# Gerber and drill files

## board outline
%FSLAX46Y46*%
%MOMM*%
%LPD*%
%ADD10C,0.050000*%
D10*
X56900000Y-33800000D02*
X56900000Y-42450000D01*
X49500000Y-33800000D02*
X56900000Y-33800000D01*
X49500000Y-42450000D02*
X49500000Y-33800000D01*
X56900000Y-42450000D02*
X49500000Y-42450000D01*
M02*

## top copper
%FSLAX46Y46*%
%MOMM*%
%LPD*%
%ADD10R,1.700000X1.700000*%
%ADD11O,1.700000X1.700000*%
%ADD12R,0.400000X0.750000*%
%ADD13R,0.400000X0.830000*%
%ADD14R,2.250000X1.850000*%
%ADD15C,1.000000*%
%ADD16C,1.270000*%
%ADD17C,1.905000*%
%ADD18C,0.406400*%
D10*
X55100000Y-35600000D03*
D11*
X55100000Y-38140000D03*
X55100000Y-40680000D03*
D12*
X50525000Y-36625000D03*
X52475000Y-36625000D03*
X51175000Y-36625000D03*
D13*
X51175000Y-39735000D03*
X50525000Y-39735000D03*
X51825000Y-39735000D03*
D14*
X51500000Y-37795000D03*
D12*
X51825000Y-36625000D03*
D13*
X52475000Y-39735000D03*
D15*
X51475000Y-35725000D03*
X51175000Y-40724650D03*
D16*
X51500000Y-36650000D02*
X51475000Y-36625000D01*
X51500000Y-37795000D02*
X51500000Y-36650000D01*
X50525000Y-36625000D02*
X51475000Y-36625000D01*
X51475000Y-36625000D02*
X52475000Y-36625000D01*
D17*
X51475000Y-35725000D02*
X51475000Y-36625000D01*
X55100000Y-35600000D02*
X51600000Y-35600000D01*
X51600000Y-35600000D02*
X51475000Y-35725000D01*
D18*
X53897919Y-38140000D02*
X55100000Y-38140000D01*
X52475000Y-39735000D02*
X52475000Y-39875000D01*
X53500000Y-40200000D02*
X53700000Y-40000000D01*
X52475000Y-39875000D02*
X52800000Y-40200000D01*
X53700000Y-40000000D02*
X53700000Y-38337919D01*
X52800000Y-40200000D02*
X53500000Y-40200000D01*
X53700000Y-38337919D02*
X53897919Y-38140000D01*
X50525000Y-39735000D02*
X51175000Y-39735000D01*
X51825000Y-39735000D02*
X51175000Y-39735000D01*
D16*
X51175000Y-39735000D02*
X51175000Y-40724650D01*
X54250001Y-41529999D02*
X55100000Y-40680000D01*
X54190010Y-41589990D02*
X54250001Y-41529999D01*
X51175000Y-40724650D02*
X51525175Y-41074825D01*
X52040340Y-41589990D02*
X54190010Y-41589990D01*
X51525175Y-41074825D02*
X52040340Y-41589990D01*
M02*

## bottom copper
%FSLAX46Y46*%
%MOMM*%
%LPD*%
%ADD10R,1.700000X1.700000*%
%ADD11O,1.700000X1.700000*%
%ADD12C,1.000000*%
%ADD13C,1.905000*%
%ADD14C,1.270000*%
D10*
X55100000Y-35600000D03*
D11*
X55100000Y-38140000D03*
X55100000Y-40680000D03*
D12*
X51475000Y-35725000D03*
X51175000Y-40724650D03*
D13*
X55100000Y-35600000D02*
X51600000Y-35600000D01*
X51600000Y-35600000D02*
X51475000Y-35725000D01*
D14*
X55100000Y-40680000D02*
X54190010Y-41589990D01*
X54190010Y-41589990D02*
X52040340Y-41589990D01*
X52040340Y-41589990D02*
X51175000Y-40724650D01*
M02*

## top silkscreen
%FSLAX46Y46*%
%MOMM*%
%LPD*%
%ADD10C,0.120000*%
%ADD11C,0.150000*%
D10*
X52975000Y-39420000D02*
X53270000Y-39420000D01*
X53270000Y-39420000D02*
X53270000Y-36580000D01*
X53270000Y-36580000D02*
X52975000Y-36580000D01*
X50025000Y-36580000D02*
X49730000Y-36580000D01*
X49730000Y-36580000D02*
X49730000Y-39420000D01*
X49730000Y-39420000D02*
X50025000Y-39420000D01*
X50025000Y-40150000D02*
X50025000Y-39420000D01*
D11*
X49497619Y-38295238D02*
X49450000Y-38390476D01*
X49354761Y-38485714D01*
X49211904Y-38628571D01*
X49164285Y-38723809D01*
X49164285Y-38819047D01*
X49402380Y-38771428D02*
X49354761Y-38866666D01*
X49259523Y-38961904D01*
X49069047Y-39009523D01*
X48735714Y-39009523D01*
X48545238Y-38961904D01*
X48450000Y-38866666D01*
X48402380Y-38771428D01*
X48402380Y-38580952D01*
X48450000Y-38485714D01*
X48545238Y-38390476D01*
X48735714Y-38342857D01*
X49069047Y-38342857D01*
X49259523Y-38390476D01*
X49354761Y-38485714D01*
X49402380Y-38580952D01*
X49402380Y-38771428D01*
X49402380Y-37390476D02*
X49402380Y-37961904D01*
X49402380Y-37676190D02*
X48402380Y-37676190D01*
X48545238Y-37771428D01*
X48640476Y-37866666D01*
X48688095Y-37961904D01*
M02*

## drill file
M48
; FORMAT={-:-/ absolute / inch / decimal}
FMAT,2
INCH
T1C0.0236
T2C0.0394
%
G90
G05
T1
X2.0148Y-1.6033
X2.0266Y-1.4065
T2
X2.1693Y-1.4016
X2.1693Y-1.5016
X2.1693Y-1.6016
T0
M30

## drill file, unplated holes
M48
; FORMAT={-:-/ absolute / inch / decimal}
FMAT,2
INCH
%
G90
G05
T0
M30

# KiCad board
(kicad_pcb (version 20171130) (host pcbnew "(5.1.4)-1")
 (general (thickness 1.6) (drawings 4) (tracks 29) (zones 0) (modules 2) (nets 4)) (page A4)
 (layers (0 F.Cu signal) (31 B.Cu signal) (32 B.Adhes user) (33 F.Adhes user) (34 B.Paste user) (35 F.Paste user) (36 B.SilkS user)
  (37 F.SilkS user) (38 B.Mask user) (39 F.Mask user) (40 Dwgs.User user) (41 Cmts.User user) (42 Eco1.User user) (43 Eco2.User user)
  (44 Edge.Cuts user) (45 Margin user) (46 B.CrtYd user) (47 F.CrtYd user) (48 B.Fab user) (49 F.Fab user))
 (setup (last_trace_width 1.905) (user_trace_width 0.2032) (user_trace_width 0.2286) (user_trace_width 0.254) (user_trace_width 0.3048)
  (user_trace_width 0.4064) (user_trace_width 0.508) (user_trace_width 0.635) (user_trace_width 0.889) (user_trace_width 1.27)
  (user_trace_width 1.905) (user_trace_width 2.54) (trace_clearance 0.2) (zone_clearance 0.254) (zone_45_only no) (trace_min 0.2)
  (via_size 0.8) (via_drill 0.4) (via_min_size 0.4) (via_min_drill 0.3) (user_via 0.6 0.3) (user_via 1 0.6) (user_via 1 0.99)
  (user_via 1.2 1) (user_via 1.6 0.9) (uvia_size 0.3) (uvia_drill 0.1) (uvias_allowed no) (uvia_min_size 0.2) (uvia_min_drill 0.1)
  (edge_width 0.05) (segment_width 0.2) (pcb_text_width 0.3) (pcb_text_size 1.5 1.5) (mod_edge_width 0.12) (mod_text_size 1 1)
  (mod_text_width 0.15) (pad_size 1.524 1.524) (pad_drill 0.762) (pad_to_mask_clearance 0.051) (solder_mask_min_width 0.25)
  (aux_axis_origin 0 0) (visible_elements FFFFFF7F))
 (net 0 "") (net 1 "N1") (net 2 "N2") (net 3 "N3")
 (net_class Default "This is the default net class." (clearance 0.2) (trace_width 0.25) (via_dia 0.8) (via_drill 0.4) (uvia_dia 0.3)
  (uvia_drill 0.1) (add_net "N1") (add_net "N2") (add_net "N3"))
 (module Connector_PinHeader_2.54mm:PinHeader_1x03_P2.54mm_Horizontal (layer B.Cu) (at 55.1 35.6 180)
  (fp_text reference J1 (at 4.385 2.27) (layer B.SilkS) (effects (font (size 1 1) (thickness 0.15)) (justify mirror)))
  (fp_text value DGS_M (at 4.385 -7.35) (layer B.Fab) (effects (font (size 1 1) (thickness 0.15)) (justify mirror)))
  (pad 1 thru_hole rect (at 0 0 180) (size 1.7 1.7) (drill 1) (layers *.Cu *.Mask) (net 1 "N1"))
  (pad 2 thru_hole oval (at 0 -2.54 180) (size 1.7 1.7) (drill 1) (layers *.Cu *.Mask) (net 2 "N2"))
  (pad 3 thru_hole oval (at 0 -5.08 180) (size 1.7 1.7) (drill 1) (layers *.Cu *.Mask) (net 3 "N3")))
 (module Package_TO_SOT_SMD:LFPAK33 (layer F.Cu) (at 51.5 38.2 90) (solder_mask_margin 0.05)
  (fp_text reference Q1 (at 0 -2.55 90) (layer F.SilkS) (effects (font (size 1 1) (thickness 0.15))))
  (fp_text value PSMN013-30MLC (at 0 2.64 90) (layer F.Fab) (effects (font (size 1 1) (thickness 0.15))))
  (fp_line (start -1.22 1.475) (end -1.22 1.77) (layer F.SilkS) (width 0.12))
  (fp_line (start -1.22 1.77) (end 1.62 1.77) (layer F.SilkS) (width 0.12))
  (fp_line (start 1.62 1.77) (end 1.62 1.475) (layer F.SilkS) (width 0.12))
  (fp_line (start 1.62 -1.475) (end 1.62 -1.77) (layer F.SilkS) (width 0.12))
  (fp_line (start 1.62 -1.77) (end -1.22 -1.77) (layer F.SilkS) (width 0.12))
  (fp_line (start -1.22 -1.77) (end -1.22 -1.475) (layer F.SilkS) (width 0.12))
  (fp_line (start -1.95 -1.475) (end -1.22 -1.475) (layer F.SilkS) (width 0.12))
  (pad "" smd rect (at -0.215 -0.626 90) (size 0.51 0.635) (layers F.Paste))
  (pad "" smd rect (at 0.645 -0.626 90) (size 0.51 0.635) (layers F.Paste))
  (pad "" smd rect (at -0.215 0.626 90) (size 0.51 0.635) (layers F.Paste))
  (pad "" smd rect (at 0.645 0.626 90) (size 0.51 0.635) (layers F.Paste))
  (pad 5 smd rect (at 1.575 -0.975 90) (size 0.75 0.4) (layers F.Cu F.Mask) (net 1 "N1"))
  (pad 5 smd rect (at 1.575 0.975 90) (size 0.75 0.4) (layers F.Cu F.Mask) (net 1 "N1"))
  (pad 5 smd rect (at 1.575 -0.325 90) (size 0.75 0.4) (layers F.Cu F.Mask) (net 1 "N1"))
  (pad 2 smd rect (at -1.535 -0.325 90) (size 0.83 0.4) (layers F.Cu F.Mask) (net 3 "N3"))
  (pad 1 smd rect (at -1.535 -0.975 90) (size 0.83 0.4) (layers F.Cu F.Mask) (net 3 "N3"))
  (pad 3 smd rect (at -1.535 0.325 90) (size 0.83 0.4) (layers F.Cu F.Mask) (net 3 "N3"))
  (pad 5 smd rect (at 0.405 0 90) (size 1.85 2.25) (layers F.Cu F.Mask) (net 1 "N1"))
  (pad "" smd rect (at -1.535 0.975 90) (size 0.83 0.3) (layers F.Paste))
  (pad 5 smd rect (at 1.575 0.325 90) (size 0.75 0.4) (layers F.Cu F.Mask) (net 1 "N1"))
  (pad 4 smd rect (at -1.535 0.975 90) (size 0.83 0.4) (layers F.Cu F.Mask) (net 2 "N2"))
  (pad "" smd rect (at -1.535 0.325 90) (size 0.83 0.3) (layers F.Paste))
  (pad "" smd rect (at -1.535 -0.325 90) (size 0.83 0.3) (layers F.Paste))
  (pad "" smd rect (at -1.535 -0.975 90) (size 0.83 0.3) (layers F.Paste))
  (pad "" smd rect (at 1.575 -0.975 90) (size 0.75 0.3) (layers F.Paste))
  (pad "" smd rect (at 1.575 -0.325 90) (size 0.75 0.3) (layers F.Paste))
  (pad "" smd rect (at 1.575 0.325 90) (size 0.75 0.3) (layers F.Paste))
  (pad "" smd rect (at 1.575 0.975 90) (size 0.75 0.3) (layers F.Paste)))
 (gr_line (start 56.9 33.8) (end 56.9 42.45) (layer Edge.Cuts) (width 0.05))
 (gr_line (start 49.5 33.8) (end 56.9 33.8) (layer Edge.Cuts) (width 0.05))
 (gr_line (start 49.5 42.45) (end 49.5 33.8) (layer Edge.Cuts) (width 0.05))
 (gr_line (start 56.9 42.45) (end 49.5 42.45) (layer Edge.Cuts) (width 0.05))
 (segment (start 51.5 36.65) (end 51.475 36.625) (width 1.27) (layer F.Cu) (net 1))
 (segment (start 51.5 37.795) (end 51.5 36.65) (width 1.27) (layer F.Cu) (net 1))
 (segment (start 50.525 36.625) (end 51.475 36.625) (width 1.27) (layer F.Cu) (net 1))
 (segment (start 51.475 36.625) (end 52.475 36.625) (width 1.27) (layer F.Cu) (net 1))
 (segment (start 51.475 35.725) (end 51.475 36.625) (width 1.905) (layer F.Cu) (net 1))
 (segment (start 55.1 35.6) (end 51.6 35.6) (width 1.905) (layer F.Cu) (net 1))
 (segment (start 51.6 35.6) (end 51.475 35.725) (width 1.905) (layer F.Cu) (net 1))
 (via (at 51.475 35.725) (size 1) (drill 0.6) (layers F.Cu B.Cu) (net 1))
 (segment (start 55.1 35.6) (end 51.6 35.6) (width 1.905) (layer B.Cu) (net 1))
 (segment (start 51.6 35.6) (end 51.475 35.725) (width 1.905) (layer B.Cu) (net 1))
 (segment (start 53.897919 38.14) (end 55.1 38.14) (width 0.4064) (layer F.Cu) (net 2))
 (segment (start 52.475 39.735) (end 52.475 39.875) (width 0.4064) (layer F.Cu) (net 2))
 (segment (start 53.5 40.2) (end 53.7 40) (width 0.4064) (layer F.Cu) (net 2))
 (segment (start 52.475 39.875) (end 52.8 40.2) (width 0.4064) (layer F.Cu) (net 2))
 (segment (start 53.7 40) (end 53.7 38.337919) (width 0.4064) (layer F.Cu) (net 2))
 (segment (start 52.8 40.2) (end 53.5 40.2) (width 0.4064) (layer F.Cu) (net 2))
 (segment (start 53.7 38.337919) (end 53.897919 38.14) (width 0.4064) (layer F.Cu) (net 2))
 (segment (start 50.525 39.735) (end 51.175 39.735) (width 0.4064) (layer F.Cu) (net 3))
 (segment (start 51.825 39.735) (end 51.175 39.735) (width 0.4064) (layer F.Cu) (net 3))
 (segment (start 51.175 39.735) (end 51.175 40.72465) (width 1.27) (layer F.Cu) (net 3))
 (segment (start 54.250001 41.529999) (end 55.1 40.68) (width 1.27) (layer F.Cu) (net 3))
 (segment (start 54.19001 41.58999) (end 54.250001 41.529999) (width 1.27) (layer F.Cu) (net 3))
 (segment (start 51.175 40.72465) (end 51.525175 41.074825) (width 1.27) (layer F.Cu) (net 3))
 (segment (start 52.04034 41.58999) (end 54.19001 41.58999) (width 1.27) (layer F.Cu) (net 3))
 (segment (start 51.525175 41.074825) (end 52.04034 41.58999) (width 1.27) (layer F.Cu) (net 3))
 (segment (start 55.1 40.68) (end 54.19001 41.58999) (width 1.27) (layer B.Cu) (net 3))
 (via (at 51.175 40.72465) (size 1) (drill 0.6) (layers F.Cu B.Cu) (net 3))
 (segment (start 54.19001 41.58999) (end 52.04034 41.58999) (width 1.27) (layer B.Cu) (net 3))
 (segment (start 52.04034 41.58999) (end 51.175 40.72465) (width 1.27) (layer B.Cu) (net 3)))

